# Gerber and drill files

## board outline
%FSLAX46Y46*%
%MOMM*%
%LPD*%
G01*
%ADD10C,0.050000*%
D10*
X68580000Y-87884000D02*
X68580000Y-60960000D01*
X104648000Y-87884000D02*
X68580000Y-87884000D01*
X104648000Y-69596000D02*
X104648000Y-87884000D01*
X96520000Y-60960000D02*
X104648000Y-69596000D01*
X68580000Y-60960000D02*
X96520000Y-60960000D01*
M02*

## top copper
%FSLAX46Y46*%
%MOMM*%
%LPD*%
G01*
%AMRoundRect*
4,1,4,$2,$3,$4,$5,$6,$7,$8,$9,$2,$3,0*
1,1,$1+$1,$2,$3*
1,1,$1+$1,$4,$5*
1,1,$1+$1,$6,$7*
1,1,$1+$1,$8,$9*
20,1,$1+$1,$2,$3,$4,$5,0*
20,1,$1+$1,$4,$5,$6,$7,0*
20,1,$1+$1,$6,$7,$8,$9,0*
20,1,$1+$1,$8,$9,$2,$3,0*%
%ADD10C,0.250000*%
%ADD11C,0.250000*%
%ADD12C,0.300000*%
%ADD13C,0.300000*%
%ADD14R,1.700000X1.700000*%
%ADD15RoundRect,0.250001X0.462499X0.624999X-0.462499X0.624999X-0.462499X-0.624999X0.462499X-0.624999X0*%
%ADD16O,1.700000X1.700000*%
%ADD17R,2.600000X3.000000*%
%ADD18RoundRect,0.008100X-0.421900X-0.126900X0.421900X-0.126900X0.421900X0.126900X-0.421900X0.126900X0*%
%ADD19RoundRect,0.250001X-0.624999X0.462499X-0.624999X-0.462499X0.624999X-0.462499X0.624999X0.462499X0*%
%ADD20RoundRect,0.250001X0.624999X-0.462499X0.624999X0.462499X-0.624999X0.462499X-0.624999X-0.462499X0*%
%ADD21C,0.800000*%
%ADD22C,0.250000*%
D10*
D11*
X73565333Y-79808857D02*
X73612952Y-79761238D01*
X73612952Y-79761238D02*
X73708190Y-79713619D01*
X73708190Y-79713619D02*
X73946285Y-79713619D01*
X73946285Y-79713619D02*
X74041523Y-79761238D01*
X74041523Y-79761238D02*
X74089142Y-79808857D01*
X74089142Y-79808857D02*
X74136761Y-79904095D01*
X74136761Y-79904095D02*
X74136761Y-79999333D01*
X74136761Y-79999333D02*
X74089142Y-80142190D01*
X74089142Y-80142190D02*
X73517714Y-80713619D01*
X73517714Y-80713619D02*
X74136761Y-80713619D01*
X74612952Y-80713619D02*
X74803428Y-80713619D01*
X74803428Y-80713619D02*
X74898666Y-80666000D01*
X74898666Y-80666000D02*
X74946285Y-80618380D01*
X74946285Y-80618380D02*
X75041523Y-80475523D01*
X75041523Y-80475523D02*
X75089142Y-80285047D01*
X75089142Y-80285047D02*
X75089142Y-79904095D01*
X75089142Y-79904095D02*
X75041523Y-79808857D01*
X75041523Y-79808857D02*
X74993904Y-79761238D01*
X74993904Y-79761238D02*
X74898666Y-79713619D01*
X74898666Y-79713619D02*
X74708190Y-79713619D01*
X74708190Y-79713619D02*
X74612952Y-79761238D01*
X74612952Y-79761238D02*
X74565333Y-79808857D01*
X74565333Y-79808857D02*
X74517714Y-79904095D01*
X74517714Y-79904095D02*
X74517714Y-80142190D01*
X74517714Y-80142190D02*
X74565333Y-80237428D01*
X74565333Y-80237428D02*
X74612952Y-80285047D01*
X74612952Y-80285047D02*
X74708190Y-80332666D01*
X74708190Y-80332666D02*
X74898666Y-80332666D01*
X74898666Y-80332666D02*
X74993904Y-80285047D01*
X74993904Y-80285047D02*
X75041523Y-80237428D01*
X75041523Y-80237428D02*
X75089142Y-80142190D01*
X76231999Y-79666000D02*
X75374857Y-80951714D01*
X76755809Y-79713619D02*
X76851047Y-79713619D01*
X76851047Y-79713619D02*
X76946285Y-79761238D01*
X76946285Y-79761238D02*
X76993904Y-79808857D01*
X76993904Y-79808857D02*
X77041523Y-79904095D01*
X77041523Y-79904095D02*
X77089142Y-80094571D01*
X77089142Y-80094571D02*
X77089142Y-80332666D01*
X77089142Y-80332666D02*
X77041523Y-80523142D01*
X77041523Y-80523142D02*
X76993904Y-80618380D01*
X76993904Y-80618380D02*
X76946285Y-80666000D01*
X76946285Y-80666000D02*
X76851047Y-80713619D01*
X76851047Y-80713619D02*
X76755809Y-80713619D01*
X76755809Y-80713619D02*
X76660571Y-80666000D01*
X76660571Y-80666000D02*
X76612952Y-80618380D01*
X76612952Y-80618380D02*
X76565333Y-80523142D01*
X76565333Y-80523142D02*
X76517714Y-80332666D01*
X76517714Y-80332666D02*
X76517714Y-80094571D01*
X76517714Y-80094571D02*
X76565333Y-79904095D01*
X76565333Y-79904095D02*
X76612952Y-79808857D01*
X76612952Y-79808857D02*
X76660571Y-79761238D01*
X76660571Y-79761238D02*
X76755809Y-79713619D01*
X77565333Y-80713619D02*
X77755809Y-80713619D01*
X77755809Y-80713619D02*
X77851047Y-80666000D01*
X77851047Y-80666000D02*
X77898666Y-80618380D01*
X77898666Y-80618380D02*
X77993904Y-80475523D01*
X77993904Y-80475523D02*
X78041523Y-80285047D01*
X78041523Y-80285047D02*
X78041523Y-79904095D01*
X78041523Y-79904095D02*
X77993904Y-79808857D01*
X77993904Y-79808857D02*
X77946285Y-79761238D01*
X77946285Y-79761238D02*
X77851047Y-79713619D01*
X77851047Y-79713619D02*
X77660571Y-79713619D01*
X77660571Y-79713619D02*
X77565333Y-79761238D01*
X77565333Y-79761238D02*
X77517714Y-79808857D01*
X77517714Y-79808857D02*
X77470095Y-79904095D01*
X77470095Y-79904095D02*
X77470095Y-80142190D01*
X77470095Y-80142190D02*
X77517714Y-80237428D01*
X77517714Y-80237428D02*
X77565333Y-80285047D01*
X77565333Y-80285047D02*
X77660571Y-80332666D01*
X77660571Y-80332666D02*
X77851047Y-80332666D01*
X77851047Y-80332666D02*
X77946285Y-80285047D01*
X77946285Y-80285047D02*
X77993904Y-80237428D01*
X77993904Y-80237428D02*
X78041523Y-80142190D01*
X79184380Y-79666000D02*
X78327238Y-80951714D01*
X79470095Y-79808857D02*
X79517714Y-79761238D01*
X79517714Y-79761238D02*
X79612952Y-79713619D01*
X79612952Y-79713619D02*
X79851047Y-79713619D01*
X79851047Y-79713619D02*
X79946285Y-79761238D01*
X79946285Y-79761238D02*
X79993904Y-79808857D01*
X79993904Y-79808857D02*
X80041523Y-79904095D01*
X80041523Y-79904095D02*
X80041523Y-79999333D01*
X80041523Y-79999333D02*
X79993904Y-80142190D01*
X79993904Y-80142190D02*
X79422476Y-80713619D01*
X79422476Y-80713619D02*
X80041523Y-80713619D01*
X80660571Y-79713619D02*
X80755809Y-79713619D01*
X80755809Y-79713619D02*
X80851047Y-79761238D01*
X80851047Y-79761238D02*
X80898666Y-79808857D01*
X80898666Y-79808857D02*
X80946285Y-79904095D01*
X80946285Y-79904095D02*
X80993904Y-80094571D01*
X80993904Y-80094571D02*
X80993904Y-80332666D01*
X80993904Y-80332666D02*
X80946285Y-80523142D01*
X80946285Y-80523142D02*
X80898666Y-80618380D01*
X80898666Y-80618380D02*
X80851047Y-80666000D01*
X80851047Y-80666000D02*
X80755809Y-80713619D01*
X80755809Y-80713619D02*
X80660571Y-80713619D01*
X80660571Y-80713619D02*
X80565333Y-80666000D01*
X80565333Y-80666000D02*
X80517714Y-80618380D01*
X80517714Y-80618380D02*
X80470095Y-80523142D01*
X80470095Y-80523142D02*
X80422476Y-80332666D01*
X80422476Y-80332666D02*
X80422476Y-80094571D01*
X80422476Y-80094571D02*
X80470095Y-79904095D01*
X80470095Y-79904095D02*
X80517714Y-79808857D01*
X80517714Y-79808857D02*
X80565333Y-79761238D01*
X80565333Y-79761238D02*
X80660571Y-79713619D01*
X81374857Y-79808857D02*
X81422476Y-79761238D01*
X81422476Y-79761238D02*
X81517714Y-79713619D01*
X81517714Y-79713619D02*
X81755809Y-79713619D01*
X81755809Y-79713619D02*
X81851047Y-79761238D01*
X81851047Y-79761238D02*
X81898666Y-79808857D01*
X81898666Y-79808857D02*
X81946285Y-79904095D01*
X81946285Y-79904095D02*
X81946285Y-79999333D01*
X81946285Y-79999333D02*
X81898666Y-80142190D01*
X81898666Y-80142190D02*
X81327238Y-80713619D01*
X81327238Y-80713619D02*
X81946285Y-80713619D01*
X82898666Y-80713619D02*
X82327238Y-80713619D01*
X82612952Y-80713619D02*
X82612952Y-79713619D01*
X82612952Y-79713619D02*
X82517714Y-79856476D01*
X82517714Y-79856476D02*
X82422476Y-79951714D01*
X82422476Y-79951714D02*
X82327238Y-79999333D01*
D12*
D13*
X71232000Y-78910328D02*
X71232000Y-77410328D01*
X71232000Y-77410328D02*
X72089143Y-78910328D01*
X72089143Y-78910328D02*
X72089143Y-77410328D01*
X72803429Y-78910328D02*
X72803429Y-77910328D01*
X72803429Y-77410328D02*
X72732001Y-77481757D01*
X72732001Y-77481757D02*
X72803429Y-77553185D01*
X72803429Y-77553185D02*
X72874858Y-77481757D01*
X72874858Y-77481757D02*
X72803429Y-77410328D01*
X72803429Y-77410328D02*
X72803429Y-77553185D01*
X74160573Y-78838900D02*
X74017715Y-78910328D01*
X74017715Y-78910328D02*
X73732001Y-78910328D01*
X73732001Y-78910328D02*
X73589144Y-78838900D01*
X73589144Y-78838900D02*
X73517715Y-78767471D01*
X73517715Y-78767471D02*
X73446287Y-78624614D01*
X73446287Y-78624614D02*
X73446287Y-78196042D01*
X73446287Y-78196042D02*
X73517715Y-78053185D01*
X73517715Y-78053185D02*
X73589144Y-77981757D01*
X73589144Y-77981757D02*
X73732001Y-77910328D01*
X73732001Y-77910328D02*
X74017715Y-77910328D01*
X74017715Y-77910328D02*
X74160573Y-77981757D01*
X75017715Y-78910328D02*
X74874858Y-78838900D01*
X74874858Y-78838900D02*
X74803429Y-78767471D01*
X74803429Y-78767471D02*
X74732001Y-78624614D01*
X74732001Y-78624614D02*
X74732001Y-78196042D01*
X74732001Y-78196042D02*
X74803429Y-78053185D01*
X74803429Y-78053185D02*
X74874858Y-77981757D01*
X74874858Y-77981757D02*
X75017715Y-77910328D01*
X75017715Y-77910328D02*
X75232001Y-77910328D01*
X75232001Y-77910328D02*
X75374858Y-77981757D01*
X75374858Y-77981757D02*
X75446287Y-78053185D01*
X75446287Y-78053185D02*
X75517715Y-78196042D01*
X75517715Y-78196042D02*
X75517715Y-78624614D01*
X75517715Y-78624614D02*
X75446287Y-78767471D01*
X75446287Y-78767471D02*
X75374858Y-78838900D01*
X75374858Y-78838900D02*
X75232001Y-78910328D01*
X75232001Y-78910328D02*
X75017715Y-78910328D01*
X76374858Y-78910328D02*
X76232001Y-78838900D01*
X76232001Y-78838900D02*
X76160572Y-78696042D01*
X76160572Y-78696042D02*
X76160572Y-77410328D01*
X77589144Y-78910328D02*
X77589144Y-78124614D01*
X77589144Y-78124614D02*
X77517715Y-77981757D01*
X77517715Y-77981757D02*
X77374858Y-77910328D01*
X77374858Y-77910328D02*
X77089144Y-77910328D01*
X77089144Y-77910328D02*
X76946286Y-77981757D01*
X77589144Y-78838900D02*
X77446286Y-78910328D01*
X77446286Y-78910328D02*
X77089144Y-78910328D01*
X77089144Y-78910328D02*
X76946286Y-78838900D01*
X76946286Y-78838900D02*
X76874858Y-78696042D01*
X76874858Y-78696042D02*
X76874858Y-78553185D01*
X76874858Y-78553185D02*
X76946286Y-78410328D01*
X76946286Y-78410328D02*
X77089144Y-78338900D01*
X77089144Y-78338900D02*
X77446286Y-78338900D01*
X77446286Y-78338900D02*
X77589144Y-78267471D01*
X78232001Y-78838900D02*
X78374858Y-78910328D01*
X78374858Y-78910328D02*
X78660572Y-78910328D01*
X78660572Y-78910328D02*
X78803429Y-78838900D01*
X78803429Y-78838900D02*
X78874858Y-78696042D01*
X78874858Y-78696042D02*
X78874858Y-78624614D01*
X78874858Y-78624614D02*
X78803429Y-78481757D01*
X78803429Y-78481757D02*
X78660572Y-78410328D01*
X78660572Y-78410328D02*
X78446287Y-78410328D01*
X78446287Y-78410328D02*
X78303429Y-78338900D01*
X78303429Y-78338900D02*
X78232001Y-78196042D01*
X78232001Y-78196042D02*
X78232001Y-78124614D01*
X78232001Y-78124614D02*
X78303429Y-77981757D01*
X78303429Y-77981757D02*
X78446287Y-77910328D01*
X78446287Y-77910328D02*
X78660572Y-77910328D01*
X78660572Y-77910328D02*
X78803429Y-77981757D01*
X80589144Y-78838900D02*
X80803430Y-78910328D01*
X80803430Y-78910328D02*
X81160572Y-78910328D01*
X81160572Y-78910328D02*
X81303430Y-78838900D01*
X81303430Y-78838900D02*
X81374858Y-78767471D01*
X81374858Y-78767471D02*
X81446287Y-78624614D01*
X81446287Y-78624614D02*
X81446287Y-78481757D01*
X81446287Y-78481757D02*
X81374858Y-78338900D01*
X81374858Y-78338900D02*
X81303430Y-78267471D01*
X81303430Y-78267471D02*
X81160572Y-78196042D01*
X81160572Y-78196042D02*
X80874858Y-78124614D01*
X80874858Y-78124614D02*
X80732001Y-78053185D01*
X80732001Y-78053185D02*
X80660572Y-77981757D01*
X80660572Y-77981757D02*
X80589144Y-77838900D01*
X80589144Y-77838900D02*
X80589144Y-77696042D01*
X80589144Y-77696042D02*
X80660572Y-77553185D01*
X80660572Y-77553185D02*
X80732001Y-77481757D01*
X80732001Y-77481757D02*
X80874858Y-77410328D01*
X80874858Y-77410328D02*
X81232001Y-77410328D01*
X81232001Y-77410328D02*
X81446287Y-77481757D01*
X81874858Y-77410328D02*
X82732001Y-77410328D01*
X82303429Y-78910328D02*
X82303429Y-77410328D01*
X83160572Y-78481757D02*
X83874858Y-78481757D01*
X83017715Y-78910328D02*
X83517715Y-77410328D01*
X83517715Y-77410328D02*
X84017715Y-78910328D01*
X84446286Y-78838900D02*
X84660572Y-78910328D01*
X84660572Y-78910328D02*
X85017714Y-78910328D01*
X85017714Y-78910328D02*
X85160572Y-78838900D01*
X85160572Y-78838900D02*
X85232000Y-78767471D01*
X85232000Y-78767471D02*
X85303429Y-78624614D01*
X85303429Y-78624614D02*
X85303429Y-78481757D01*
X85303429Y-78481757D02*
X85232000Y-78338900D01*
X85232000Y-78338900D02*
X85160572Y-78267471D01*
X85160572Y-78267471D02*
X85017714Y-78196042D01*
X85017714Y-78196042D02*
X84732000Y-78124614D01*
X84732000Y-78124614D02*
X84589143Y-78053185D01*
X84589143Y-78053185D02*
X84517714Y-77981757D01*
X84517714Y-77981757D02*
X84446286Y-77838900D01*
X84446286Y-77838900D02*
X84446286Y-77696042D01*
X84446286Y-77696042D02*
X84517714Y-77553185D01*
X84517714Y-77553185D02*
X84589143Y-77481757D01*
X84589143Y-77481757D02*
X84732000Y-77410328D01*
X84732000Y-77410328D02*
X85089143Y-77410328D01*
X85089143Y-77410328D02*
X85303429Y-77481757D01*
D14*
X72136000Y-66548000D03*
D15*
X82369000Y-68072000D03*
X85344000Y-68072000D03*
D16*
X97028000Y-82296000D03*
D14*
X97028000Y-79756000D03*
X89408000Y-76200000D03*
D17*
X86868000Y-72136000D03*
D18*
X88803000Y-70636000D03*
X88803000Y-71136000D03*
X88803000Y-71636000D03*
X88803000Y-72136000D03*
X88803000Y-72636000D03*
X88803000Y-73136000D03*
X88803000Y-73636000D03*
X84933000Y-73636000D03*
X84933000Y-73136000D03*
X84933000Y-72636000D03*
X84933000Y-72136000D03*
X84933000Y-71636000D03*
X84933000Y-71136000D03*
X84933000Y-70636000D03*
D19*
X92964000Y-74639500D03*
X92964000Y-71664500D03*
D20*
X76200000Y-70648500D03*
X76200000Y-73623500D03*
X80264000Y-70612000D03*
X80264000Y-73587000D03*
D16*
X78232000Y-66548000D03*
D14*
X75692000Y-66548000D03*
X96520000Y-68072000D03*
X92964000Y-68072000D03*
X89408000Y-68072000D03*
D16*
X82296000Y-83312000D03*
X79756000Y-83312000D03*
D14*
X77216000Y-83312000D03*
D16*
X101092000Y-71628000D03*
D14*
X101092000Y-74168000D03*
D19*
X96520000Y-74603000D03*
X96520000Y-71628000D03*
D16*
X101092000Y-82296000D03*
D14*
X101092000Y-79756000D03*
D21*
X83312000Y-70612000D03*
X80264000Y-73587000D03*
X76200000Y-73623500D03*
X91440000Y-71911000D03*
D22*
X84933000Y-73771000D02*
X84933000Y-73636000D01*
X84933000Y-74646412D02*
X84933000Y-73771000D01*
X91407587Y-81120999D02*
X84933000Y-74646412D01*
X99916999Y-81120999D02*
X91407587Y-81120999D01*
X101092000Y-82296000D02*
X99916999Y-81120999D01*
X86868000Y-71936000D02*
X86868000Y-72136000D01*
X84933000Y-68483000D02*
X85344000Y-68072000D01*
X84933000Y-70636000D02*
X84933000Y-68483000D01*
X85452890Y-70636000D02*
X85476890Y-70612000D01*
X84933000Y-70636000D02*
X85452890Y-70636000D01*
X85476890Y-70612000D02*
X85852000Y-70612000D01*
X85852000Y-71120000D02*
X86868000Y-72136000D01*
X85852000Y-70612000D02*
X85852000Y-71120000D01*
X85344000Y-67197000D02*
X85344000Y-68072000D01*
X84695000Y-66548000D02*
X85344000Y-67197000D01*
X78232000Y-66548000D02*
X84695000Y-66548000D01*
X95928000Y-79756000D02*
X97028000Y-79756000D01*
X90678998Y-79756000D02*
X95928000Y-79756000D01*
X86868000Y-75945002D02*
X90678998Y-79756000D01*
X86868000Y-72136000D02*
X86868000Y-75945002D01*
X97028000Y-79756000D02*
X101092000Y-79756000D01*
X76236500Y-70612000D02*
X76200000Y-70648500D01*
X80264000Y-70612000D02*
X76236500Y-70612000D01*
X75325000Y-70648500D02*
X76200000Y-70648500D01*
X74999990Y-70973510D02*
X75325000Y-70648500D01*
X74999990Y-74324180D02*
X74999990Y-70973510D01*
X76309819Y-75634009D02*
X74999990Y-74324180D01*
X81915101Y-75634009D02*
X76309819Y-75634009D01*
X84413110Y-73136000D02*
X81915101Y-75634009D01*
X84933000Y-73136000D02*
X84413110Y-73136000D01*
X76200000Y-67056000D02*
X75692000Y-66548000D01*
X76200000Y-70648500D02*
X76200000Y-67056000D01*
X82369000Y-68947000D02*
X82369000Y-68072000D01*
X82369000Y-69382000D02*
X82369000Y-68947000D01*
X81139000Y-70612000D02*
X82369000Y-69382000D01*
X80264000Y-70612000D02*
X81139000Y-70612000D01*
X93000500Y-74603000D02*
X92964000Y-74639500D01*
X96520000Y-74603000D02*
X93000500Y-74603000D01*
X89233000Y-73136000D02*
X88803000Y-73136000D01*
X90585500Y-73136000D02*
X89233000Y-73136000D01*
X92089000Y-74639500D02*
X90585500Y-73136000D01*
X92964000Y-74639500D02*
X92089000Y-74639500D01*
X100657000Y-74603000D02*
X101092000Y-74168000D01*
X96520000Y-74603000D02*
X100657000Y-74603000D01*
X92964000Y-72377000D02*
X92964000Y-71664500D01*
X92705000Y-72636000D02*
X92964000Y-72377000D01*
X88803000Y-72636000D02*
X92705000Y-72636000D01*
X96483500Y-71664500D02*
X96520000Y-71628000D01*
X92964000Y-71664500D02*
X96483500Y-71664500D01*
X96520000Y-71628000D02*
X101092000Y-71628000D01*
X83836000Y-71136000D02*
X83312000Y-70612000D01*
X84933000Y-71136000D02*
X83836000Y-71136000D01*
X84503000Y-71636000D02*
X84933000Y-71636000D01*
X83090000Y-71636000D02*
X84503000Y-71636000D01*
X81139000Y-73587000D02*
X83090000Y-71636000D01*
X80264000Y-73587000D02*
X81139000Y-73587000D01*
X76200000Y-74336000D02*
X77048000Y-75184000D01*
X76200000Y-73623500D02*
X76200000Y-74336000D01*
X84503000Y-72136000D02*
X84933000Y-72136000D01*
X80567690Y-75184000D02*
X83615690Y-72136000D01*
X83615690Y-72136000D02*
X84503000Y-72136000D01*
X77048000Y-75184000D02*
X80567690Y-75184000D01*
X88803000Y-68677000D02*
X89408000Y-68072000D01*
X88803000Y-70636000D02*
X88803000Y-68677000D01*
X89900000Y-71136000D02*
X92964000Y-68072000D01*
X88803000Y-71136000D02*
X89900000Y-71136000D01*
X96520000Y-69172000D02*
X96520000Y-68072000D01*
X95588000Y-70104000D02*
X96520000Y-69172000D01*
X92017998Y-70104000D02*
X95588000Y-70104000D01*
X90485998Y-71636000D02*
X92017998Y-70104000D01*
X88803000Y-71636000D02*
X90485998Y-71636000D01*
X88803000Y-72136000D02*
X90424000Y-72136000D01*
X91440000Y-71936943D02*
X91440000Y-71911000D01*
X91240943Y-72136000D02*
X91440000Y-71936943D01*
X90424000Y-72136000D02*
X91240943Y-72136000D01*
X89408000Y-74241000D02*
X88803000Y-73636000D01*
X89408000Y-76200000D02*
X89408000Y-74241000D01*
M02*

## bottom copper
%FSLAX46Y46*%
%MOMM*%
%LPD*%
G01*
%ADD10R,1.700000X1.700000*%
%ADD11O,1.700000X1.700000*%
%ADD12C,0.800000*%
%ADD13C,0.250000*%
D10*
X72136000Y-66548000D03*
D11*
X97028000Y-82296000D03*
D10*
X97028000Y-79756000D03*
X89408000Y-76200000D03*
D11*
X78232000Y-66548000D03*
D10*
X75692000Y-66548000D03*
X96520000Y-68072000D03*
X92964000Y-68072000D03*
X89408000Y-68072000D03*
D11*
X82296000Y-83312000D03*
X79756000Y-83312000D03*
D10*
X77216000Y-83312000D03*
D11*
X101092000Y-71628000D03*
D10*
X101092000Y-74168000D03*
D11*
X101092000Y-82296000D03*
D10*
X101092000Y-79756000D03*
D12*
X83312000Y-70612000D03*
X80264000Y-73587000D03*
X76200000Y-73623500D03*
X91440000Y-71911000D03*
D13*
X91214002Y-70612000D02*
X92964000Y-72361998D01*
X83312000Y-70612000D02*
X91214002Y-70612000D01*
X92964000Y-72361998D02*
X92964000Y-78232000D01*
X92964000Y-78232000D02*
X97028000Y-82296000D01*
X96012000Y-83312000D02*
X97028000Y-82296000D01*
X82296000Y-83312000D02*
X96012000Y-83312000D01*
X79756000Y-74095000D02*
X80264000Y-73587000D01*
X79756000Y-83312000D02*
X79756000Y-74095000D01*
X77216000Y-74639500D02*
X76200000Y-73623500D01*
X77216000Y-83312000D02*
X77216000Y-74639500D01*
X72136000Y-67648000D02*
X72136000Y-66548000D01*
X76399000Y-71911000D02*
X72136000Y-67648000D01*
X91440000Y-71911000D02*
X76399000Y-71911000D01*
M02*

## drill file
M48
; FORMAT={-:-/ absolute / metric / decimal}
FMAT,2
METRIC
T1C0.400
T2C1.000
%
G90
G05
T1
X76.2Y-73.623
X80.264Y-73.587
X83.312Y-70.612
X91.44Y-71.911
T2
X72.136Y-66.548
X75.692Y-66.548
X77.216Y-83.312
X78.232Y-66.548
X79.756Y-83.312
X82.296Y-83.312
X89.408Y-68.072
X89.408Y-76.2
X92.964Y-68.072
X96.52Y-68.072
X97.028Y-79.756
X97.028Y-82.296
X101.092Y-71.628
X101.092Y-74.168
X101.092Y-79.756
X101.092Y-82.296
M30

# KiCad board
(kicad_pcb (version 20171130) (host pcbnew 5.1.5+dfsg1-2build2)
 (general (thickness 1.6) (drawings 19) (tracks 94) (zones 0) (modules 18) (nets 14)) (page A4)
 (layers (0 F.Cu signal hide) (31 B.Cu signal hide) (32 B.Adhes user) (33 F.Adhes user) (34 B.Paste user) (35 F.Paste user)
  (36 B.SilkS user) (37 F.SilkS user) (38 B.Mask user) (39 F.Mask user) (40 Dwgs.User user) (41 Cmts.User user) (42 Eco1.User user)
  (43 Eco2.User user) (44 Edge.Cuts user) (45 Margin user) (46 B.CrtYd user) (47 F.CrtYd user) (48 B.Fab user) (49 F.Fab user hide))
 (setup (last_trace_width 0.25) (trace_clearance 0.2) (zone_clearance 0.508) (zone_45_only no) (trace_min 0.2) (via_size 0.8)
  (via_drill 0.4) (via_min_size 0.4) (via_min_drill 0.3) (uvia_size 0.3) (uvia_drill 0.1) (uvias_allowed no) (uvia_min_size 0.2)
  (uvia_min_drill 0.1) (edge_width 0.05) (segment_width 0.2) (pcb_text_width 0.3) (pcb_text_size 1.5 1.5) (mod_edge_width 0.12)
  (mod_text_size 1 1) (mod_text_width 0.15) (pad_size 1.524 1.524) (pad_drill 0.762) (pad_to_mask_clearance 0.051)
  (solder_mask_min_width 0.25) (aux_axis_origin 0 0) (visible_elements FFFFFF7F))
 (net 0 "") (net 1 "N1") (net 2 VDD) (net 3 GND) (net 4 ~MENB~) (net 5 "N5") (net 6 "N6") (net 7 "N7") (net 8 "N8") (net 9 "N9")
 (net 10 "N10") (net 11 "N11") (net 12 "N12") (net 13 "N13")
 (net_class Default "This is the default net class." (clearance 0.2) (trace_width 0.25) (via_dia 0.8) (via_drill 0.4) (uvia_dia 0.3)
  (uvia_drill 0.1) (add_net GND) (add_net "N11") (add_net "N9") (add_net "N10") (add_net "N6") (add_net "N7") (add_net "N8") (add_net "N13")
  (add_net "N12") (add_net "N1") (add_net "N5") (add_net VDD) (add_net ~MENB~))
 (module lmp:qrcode (layer B.Cu) (at 82.296 74.676 90)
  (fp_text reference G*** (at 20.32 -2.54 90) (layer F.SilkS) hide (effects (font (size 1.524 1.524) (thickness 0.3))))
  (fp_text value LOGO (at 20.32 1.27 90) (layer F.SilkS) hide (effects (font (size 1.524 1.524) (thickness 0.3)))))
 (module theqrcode (layer F.Cu) (at 0 0)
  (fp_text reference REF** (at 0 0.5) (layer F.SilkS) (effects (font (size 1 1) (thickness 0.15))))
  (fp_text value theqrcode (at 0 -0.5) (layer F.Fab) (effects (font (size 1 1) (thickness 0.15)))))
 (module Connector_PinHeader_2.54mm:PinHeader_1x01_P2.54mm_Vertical (layer F.Cu) (at 72.136 66.548)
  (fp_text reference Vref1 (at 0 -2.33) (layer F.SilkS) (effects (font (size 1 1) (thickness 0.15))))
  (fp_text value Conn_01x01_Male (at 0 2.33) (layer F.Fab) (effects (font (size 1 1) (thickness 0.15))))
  (pad 1 thru_hole rect (at 0 0) (size 1.7 1.7) (drill 1) (layers *.Cu *.Mask) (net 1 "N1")))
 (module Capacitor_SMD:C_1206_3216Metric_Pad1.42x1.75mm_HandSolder (layer F.Cu) (at 83.8565 68.072 180)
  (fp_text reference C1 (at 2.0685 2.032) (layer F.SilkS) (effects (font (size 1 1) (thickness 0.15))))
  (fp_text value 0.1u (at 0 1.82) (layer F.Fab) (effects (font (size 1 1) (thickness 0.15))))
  (pad 2 smd roundrect (at 1.4875 0 180) (size 1.425 1.75) (layers F.Cu F.Paste F.Mask) (roundrect_rratio 0.175439) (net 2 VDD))
  (pad 1 smd roundrect (at -1.4875 0 180) (size 1.425 1.75) (layers F.Cu F.Paste F.Mask) (roundrect_rratio 0.175439) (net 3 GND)))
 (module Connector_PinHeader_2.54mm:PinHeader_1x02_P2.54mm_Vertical (layer F.Cu) (at 97.028 79.756)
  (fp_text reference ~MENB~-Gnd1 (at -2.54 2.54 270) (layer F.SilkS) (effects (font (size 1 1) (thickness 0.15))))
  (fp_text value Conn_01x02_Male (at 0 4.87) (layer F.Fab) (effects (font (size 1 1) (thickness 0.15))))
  (pad 2 thru_hole oval (at 0 2.54) (size 1.7 1.7) (drill 1) (layers *.Cu *.Mask) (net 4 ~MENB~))
  (pad 1 thru_hole rect (at 0 0) (size 1.7 1.7) (drill 1) (layers *.Cu *.Mask) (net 3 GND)))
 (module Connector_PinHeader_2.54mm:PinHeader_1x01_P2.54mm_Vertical (layer F.Cu) (at 89.408 76.2)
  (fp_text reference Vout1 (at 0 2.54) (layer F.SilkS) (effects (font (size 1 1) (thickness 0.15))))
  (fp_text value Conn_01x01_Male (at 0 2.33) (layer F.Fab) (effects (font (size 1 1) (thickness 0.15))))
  (pad 1 thru_hole rect (at 0 0) (size 1.7 1.7) (drill 1) (layers *.Cu *.Mask) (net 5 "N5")))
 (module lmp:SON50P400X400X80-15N (layer F.Cu) (at 86.868 72.136)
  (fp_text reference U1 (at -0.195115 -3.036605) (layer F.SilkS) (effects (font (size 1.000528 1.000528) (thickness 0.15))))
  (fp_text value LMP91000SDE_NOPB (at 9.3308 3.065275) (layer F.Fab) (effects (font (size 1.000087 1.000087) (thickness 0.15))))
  (pad 15 smd rect (at 0 0) (size 2.6 3) (layers F.Cu F.Mask) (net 3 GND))
  (pad 14 smd roundrect (at 1.935 -1.5) (size 0.86 0.27) (layers F.Cu F.Paste F.Mask) (roundrect_rratio 0.03) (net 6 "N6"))
  (pad 13 smd roundrect (at 1.935 -1) (size 0.86 0.27) (layers F.Cu F.Paste F.Mask) (roundrect_rratio 0.03) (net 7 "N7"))
  (pad 12 smd roundrect (at 1.935 -0.5) (size 0.86 0.27) (layers F.Cu F.Paste F.Mask) (roundrect_rratio 0.03) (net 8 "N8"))
  (pad 11 smd roundrect (at 1.935 0) (size 0.86 0.27) (layers F.Cu F.Paste F.Mask) (roundrect_rratio 0.03) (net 1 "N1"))
  (pad 10 smd roundrect (at 1.935 0.5) (size 0.86 0.27) (layers F.Cu F.Paste F.Mask) (roundrect_rratio 0.03) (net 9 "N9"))
  (pad 9 smd roundrect (at 1.935 1) (size 0.86 0.27) (layers F.Cu F.Paste F.Mask) (roundrect_rratio 0.03) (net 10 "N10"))
  (pad 8 smd roundrect (at 1.935 1.5) (size 0.86 0.27) (layers F.Cu F.Paste F.Mask) (roundrect_rratio 0.03) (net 5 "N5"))
  (pad 7 smd roundrect (at -1.935 1.5) (size 0.86 0.27) (layers F.Cu F.Paste F.Mask) (roundrect_rratio 0.03) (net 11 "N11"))
  (pad 6 smd roundrect (at -1.935 1) (size 0.86 0.27) (layers F.Cu F.Paste F.Mask) (roundrect_rratio 0.03) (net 2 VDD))
  (pad 5 smd roundrect (at -1.935 0.5) (size 0.86 0.27) (layers F.Cu F.Paste F.Mask) (roundrect_rratio 0.03))
  (pad 4 smd roundrect (at -1.935 0) (size 0.86 0.27) (layers F.Cu F.Paste F.Mask) (roundrect_rratio 0.03) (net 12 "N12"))
  (pad 3 smd roundrect (at -1.935 -0.5) (size 0.86 0.27) (layers F.Cu F.Paste F.Mask) (roundrect_rratio 0.03) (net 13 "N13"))
  (pad 2 smd roundrect (at -1.935 -1) (size 0.86 0.27) (layers F.Cu F.Paste F.Mask) (roundrect_rratio 0.03) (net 4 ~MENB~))
  (pad 1 smd roundrect (at -1.935 -1.5) (size 0.86 0.27) (layers F.Cu F.Paste F.Mask) (roundrect_rratio 0.03) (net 3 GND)))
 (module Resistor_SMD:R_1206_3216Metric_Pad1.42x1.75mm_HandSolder (layer F.Cu) (at 92.964 73.152 270)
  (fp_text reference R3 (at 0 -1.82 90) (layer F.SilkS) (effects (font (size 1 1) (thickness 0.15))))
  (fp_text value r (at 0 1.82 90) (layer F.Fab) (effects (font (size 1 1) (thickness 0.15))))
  (pad 2 smd roundrect (at 1.4875 0 270) (size 1.425 1.75) (layers F.Cu F.Paste F.Mask) (roundrect_rratio 0.175439) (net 10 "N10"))
  (pad 1 smd roundrect (at -1.4875 0 270) (size 1.425 1.75) (layers F.Cu F.Paste F.Mask) (roundrect_rratio 0.175439) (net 9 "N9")))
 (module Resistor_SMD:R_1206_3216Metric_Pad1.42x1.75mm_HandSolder (layer F.Cu) (at 76.2 72.136 90)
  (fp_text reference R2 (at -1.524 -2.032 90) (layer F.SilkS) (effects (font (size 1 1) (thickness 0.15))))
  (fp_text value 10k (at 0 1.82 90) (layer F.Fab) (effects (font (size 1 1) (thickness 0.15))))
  (pad 2 smd roundrect (at 1.4875 0 90) (size 1.425 1.75) (layers F.Cu F.Paste F.Mask) (roundrect_rratio 0.175439) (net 2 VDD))
  (pad 1 smd roundrect (at -1.4875 0 90) (size 1.425 1.75) (layers F.Cu F.Paste F.Mask) (roundrect_rratio 0.175439) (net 12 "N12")))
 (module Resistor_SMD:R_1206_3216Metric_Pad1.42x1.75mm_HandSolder (layer F.Cu) (at 80.264 72.0995 90)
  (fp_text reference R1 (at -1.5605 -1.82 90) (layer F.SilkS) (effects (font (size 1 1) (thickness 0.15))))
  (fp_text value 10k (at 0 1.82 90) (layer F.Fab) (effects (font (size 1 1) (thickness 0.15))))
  (pad 2 smd roundrect (at 1.4875 0 90) (size 1.425 1.75) (layers F.Cu F.Paste F.Mask) (roundrect_rratio 0.175439) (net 2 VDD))
  (pad 1 smd roundrect (at -1.4875 0 90) (size 1.425 1.75) (layers F.Cu F.Paste F.Mask) (roundrect_rratio 0.175439) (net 13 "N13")))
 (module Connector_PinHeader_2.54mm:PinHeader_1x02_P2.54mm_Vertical (layer F.Cu) (at 75.692 66.548 90)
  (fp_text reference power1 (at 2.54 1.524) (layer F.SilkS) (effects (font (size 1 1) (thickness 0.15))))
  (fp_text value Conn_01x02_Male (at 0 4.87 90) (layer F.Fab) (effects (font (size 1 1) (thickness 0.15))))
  (pad 2 thru_hole oval (at 0 2.54 90) (size 1.7 1.7) (drill 1) (layers *.Cu *.Mask) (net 3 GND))
  (pad 1 thru_hole rect (at 0 0 90) (size 1.7 1.7) (drill 1) (layers *.Cu *.Mask) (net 2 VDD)))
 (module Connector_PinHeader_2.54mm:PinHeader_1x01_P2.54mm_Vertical (layer F.Cu) (at 96.52 68.072)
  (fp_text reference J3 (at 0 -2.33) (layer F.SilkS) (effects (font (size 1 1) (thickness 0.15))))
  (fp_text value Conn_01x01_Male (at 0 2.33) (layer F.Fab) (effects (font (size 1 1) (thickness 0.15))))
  (pad 1 thru_hole rect (at 0 0) (size 1.7 1.7) (drill 1) (layers *.Cu *.Mask) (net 8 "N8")))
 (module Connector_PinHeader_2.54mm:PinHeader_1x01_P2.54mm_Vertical (layer F.Cu) (at 92.964 68.072)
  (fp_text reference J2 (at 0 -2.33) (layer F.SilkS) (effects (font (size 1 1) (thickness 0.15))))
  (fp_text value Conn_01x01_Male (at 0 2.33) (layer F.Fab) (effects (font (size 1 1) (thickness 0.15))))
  (pad 1 thru_hole rect (at 0 0) (size 1.7 1.7) (drill 1) (layers *.Cu *.Mask) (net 7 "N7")))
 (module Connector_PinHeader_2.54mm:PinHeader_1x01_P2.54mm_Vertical (layer F.Cu) (at 89.408 68.072)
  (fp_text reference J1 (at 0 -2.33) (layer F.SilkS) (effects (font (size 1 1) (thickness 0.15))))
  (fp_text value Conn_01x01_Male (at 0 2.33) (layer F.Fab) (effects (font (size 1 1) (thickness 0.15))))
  (pad 1 thru_hole rect (at 0 0) (size 1.7 1.7) (drill 1) (layers *.Cu *.Mask) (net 6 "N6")))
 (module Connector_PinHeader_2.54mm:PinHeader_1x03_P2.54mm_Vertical (layer F.Cu) (at 77.216 83.312 90)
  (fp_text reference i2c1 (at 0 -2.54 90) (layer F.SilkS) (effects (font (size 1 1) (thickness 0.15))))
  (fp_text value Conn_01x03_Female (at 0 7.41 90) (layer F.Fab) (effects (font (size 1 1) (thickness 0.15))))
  (pad 3 thru_hole oval (at 0 5.08 90) (size 1.7 1.7) (drill 1) (layers *.Cu *.Mask) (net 4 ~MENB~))
  (pad 2 thru_hole oval (at 0 2.54 90) (size 1.7 1.7) (drill 1) (layers *.Cu *.Mask) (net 13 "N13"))
  (pad 1 thru_hole rect (at 0 0 90) (size 1.7 1.7) (drill 1) (layers *.Cu *.Mask) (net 12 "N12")))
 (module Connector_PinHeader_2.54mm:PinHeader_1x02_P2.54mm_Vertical (layer F.Cu) (at 101.092 74.168 180)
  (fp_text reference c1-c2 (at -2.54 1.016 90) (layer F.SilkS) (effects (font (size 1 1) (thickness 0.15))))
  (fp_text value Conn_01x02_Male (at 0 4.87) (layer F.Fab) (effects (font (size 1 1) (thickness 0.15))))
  (pad 2 thru_hole oval (at 0 2.54 180) (size 1.7 1.7) (drill 1) (layers *.Cu *.Mask) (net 9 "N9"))
  (pad 1 thru_hole rect (at 0 0 180) (size 1.7 1.7) (drill 1) (layers *.Cu *.Mask) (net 10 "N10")))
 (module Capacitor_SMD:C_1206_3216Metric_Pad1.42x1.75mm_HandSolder (layer F.Cu) (at 96.52 73.1155 270)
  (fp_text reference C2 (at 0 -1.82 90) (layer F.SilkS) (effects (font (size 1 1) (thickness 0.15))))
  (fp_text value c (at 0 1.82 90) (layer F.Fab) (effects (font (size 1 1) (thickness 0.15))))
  (pad 2 smd roundrect (at 1.4875 0 270) (size 1.425 1.75) (layers F.Cu F.Paste F.Mask) (roundrect_rratio 0.175439) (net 10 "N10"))
  (pad 1 smd roundrect (at -1.4875 0 270) (size 1.425 1.75) (layers F.Cu F.Paste F.Mask) (roundrect_rratio 0.175439) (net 9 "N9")))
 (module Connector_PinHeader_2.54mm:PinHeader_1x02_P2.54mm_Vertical (layer F.Cu) (at 101.092 79.756)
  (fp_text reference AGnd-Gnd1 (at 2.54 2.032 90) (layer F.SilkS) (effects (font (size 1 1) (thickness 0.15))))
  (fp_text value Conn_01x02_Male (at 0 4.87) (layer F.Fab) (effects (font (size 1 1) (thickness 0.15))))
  (pad 2 thru_hole oval (at 0 2.54) (size 1.7 1.7) (drill 1) (layers *.Cu *.Mask) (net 11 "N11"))
  (pad 1 thru_hole rect (at 0 0) (size 1.7 1.7) (drill 1) (layers *.Cu *.Mask) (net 3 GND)))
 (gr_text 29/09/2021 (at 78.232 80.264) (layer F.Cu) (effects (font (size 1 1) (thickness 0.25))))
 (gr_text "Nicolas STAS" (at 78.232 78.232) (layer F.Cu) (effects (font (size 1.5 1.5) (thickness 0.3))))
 (gr_line (start 68.58 87.884) (end 68.58 60.96) (layer Edge.Cuts) (width 0.05))
 (gr_line (start 104.648 87.884) (end 68.58 87.884) (layer Edge.Cuts) (width 0.05))
 (gr_line (start 104.648 69.596) (end 104.648 87.884) (layer Edge.Cuts) (width 0.05))
 (gr_line (start 96.52 60.96) (end 104.648 69.596) (layer Edge.Cuts) (width 0.05))
 (gr_line (start 68.58 60.96) (end 96.52 60.96) (layer Edge.Cuts) (width 0.05))
 (segment (start 84.933 73.771) (end 84.933 73.636) (width 0.25) (layer F.Cu) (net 11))
 (segment (start 84.933 74.646412) (end 84.933 73.771) (width 0.25) (layer F.Cu) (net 11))
 (segment (start 91.407587 81.120999) (end 84.933 74.646412) (width 0.25) (layer F.Cu) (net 11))
 (segment (start 99.916999 81.120999) (end 91.407587 81.120999) (width 0.25) (layer F.Cu) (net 11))
 (segment (start 101.092 82.296) (end 99.916999 81.120999) (width 0.25) (layer F.Cu) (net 11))
 (segment (start 86.868 71.936) (end 86.868 72.136) (width 0.25) (layer F.Cu) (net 3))
 (segment (start 84.933 68.483) (end 85.344 68.072) (width 0.25) (layer F.Cu) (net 3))
 (segment (start 84.933 70.636) (end 84.933 68.483) (width 0.25) (layer F.Cu) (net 3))
 (segment (start 85.45289 70.636) (end 85.47689 70.612) (width 0.25) (layer F.Cu) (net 3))
 (segment (start 84.933 70.636) (end 85.45289 70.636) (width 0.25) (layer F.Cu) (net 3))
 (segment (start 85.47689 70.612) (end 85.852 70.612) (width 0.25) (layer F.Cu) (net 3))
 (segment (start 85.852 71.12) (end 86.868 72.136) (width 0.25) (layer F.Cu) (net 3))
 (segment (start 85.852 70.612) (end 85.852 71.12) (width 0.25) (layer F.Cu) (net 3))
 (segment (start 85.344 67.197) (end 85.344 68.072) (width 0.25) (layer F.Cu) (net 3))
 (segment (start 84.695 66.548) (end 85.344 67.197) (width 0.25) (layer F.Cu) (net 3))
 (segment (start 78.232 66.548) (end 84.695 66.548) (width 0.25) (layer F.Cu) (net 3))
 (segment (start 95.928 79.756) (end 97.028 79.756) (width 0.25) (layer F.Cu) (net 3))
 (segment (start 90.678998 79.756) (end 95.928 79.756) (width 0.25) (layer F.Cu) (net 3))
 (segment (start 86.868 75.945002) (end 90.678998 79.756) (width 0.25) (layer F.Cu) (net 3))
 (segment (start 86.868 72.136) (end 86.868 75.945002) (width 0.25) (layer F.Cu) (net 3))
 (segment (start 97.028 79.756) (end 101.092 79.756) (width 0.25) (layer F.Cu) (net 3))
 (segment (start 76.2365 70.612) (end 76.2 70.6485) (width 0.25) (layer F.Cu) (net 2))
 (segment (start 80.264 70.612) (end 76.2365 70.612) (width 0.25) (layer F.Cu) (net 2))
 (segment (start 75.325 70.6485) (end 76.2 70.6485) (width 0.25) (layer F.Cu) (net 2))
 (segment (start 74.99999 70.97351) (end 75.325 70.6485) (width 0.25) (layer F.Cu) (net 2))
 (segment (start 74.99999 74.32418) (end 74.99999 70.97351) (width 0.25) (layer F.Cu) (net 2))
 (segment (start 76.309819 75.634009) (end 74.99999 74.32418) (width 0.25) (layer F.Cu) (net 2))
 (segment (start 81.915101 75.634009) (end 76.309819 75.634009) (width 0.25) (layer F.Cu) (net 2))
 (segment (start 84.41311 73.136) (end 81.915101 75.634009) (width 0.25) (layer F.Cu) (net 2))
 (segment (start 84.933 73.136) (end 84.41311 73.136) (width 0.25) (layer F.Cu) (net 2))
 (segment (start 76.2 67.056) (end 75.692 66.548) (width 0.25) (layer F.Cu) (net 2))
 (segment (start 76.2 70.6485) (end 76.2 67.056) (width 0.25) (layer F.Cu) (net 2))
 (segment (start 82.369 68.947) (end 82.369 68.072) (width 0.25) (layer F.Cu) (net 2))
 (segment (start 82.369 69.382) (end 82.369 68.947) (width 0.25) (layer F.Cu) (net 2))
 (segment (start 81.139 70.612) (end 82.369 69.382) (width 0.25) (layer F.Cu) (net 2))
 (segment (start 80.264 70.612) (end 81.139 70.612) (width 0.25) (layer F.Cu) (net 2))
 (segment (start 93.0005 74.603) (end 92.964 74.6395) (width 0.25) (layer F.Cu) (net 10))
 (segment (start 96.52 74.603) (end 93.0005 74.603) (width 0.25) (layer F.Cu) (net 10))
 (segment (start 89.233 73.136) (end 88.803 73.136) (width 0.25) (layer F.Cu) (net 10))
 (segment (start 90.5855 73.136) (end 89.233 73.136) (width 0.25) (layer F.Cu) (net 10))
 (segment (start 92.089 74.6395) (end 90.5855 73.136) (width 0.25) (layer F.Cu) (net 10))
 (segment (start 92.964 74.6395) (end 92.089 74.6395) (width 0.25) (layer F.Cu) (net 10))
 (segment (start 100.657 74.603) (end 101.092 74.168) (width 0.25) (layer F.Cu) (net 10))
 (segment (start 96.52 74.603) (end 100.657 74.603) (width 0.25) (layer F.Cu) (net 10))
 (segment (start 92.964 72.377) (end 92.964 71.6645) (width 0.25) (layer F.Cu) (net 9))
 (segment (start 92.705 72.636) (end 92.964 72.377) (width 0.25) (layer F.Cu) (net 9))
 (segment (start 88.803 72.636) (end 92.705 72.636) (width 0.25) (layer F.Cu) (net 9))
 (segment (start 96.4835 71.6645) (end 96.52 71.628) (width 0.25) (layer F.Cu) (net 9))
 (segment (start 92.964 71.6645) (end 96.4835 71.6645) (width 0.25) (layer F.Cu) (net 9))
 (segment (start 96.52 71.628) (end 101.092 71.628) (width 0.25) (layer F.Cu) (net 9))
 (via (at 83.312 70.612) (size 0.8) (drill 0.4) (layers F.Cu B.Cu) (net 4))
 (segment (start 83.836 71.136) (end 83.312 70.612) (width 0.25) (layer F.Cu) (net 4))
 (segment (start 84.933 71.136) (end 83.836 71.136) (width 0.25) (layer F.Cu) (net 4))
 (segment (start 91.214002 70.612) (end 92.964 72.361998) (width 0.25) (layer B.Cu) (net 4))
 (segment (start 83.312 70.612) (end 91.214002 70.612) (width 0.25) (layer B.Cu) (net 4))
 (segment (start 92.964 72.361998) (end 92.964 78.232) (width 0.25) (layer B.Cu) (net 4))
 (segment (start 92.964 78.232) (end 97.028 82.296) (width 0.25) (layer B.Cu) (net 4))
 (segment (start 96.012 83.312) (end 97.028 82.296) (width 0.25) (layer B.Cu) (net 4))
 (segment (start 82.296 83.312) (end 96.012 83.312) (width 0.25) (layer B.Cu) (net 4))
 (segment (start 84.503 71.636) (end 84.933 71.636) (width 0.25) (layer F.Cu) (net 13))
 (segment (start 83.09 71.636) (end 84.503 71.636) (width 0.25) (layer F.Cu) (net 13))
 (segment (start 81.139 73.587) (end 83.09 71.636) (width 0.25) (layer F.Cu) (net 13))
 (segment (start 80.264 73.587) (end 81.139 73.587) (width 0.25) (layer F.Cu) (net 13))
 (via (at 80.264 73.587) (size 0.8) (drill 0.4) (layers F.Cu B.Cu) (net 13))
 (segment (start 79.756 74.095) (end 80.264 73.587) (width 0.25) (layer B.Cu) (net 13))
 (segment (start 79.756 83.312) (end 79.756 74.095) (width 0.25) (layer B.Cu) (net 13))
 (segment (start 76.2 74.336) (end 77.048 75.184) (width 0.25) (layer F.Cu) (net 12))
 (segment (start 76.2 73.6235) (end 76.2 74.336) (width 0.25) (layer F.Cu) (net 12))
 (segment (start 84.503 72.136) (end 84.933 72.136) (width 0.25) (layer F.Cu) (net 12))
 (segment (start 80.56769 75.184) (end 83.61569 72.136) (width 0.25) (layer F.Cu) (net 12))
 (segment (start 83.61569 72.136) (end 84.503 72.136) (width 0.25) (layer F.Cu) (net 12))
 (segment (start 77.048 75.184) (end 80.56769 75.184) (width 0.25) (layer F.Cu) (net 12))
 (via (at 76.2 73.6235) (size 0.8) (drill 0.4) (layers F.Cu B.Cu) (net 12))
 (segment (start 77.216 74.6395) (end 76.2 73.6235) (width 0.25) (layer B.Cu) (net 12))
 (segment (start 77.216 83.312) (end 77.216 74.6395) (width 0.25) (layer B.Cu) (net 12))
 (segment (start 88.803 68.677) (end 89.408 68.072) (width 0.25) (layer F.Cu) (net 6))
 (segment (start 88.803 70.636) (end 88.803 68.677) (width 0.25) (layer F.Cu) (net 6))
 (segment (start 89.9 71.136) (end 92.964 68.072) (width 0.25) (layer F.Cu) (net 7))
 (segment (start 88.803 71.136) (end 89.9 71.136) (width 0.25) (layer F.Cu) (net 7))
 (segment (start 96.52 69.172) (end 96.52 68.072) (width 0.25) (layer F.Cu) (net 8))
 (segment (start 95.588 70.104) (end 96.52 69.172) (width 0.25) (layer F.Cu) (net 8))
 (segment (start 92.017998 70.104) (end 95.588 70.104) (width 0.25) (layer F.Cu) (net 8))
 (segment (start 90.485998 71.636) (end 92.017998 70.104) (width 0.25) (layer F.Cu) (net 8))
 (segment (start 88.803 71.636) (end 90.485998 71.636) (width 0.25) (layer F.Cu) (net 8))
 (segment (start 88.803 72.136) (end 90.424 72.136) (width 0.25) (layer F.Cu) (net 1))
 (via (at 91.44 71.911) (size 0.8) (drill 0.4) (layers F.Cu B.Cu) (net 1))
 (segment (start 91.44 71.936943) (end 91.44 71.911) (width 0.25) (layer F.Cu) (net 1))
 (segment (start 91.240943 72.136) (end 91.44 71.936943) (width 0.25) (layer F.Cu) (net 1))
 (segment (start 90.424 72.136) (end 91.240943 72.136) (width 0.25) (layer F.Cu) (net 1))
 (segment (start 72.136 67.648) (end 72.136 66.548) (width 0.25) (layer B.Cu) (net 1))
 (segment (start 76.399 71.911) (end 72.136 67.648) (width 0.25) (layer B.Cu) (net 1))
 (segment (start 91.44 71.911) (end 76.399 71.911) (width 0.25) (layer B.Cu) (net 1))
 (segment (start 89.408 74.241) (end 88.803 73.636) (width 0.25) (layer F.Cu) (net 5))
 (segment (start 89.408 76.2) (end 89.408 74.241) (width 0.25) (layer F.Cu) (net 5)))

